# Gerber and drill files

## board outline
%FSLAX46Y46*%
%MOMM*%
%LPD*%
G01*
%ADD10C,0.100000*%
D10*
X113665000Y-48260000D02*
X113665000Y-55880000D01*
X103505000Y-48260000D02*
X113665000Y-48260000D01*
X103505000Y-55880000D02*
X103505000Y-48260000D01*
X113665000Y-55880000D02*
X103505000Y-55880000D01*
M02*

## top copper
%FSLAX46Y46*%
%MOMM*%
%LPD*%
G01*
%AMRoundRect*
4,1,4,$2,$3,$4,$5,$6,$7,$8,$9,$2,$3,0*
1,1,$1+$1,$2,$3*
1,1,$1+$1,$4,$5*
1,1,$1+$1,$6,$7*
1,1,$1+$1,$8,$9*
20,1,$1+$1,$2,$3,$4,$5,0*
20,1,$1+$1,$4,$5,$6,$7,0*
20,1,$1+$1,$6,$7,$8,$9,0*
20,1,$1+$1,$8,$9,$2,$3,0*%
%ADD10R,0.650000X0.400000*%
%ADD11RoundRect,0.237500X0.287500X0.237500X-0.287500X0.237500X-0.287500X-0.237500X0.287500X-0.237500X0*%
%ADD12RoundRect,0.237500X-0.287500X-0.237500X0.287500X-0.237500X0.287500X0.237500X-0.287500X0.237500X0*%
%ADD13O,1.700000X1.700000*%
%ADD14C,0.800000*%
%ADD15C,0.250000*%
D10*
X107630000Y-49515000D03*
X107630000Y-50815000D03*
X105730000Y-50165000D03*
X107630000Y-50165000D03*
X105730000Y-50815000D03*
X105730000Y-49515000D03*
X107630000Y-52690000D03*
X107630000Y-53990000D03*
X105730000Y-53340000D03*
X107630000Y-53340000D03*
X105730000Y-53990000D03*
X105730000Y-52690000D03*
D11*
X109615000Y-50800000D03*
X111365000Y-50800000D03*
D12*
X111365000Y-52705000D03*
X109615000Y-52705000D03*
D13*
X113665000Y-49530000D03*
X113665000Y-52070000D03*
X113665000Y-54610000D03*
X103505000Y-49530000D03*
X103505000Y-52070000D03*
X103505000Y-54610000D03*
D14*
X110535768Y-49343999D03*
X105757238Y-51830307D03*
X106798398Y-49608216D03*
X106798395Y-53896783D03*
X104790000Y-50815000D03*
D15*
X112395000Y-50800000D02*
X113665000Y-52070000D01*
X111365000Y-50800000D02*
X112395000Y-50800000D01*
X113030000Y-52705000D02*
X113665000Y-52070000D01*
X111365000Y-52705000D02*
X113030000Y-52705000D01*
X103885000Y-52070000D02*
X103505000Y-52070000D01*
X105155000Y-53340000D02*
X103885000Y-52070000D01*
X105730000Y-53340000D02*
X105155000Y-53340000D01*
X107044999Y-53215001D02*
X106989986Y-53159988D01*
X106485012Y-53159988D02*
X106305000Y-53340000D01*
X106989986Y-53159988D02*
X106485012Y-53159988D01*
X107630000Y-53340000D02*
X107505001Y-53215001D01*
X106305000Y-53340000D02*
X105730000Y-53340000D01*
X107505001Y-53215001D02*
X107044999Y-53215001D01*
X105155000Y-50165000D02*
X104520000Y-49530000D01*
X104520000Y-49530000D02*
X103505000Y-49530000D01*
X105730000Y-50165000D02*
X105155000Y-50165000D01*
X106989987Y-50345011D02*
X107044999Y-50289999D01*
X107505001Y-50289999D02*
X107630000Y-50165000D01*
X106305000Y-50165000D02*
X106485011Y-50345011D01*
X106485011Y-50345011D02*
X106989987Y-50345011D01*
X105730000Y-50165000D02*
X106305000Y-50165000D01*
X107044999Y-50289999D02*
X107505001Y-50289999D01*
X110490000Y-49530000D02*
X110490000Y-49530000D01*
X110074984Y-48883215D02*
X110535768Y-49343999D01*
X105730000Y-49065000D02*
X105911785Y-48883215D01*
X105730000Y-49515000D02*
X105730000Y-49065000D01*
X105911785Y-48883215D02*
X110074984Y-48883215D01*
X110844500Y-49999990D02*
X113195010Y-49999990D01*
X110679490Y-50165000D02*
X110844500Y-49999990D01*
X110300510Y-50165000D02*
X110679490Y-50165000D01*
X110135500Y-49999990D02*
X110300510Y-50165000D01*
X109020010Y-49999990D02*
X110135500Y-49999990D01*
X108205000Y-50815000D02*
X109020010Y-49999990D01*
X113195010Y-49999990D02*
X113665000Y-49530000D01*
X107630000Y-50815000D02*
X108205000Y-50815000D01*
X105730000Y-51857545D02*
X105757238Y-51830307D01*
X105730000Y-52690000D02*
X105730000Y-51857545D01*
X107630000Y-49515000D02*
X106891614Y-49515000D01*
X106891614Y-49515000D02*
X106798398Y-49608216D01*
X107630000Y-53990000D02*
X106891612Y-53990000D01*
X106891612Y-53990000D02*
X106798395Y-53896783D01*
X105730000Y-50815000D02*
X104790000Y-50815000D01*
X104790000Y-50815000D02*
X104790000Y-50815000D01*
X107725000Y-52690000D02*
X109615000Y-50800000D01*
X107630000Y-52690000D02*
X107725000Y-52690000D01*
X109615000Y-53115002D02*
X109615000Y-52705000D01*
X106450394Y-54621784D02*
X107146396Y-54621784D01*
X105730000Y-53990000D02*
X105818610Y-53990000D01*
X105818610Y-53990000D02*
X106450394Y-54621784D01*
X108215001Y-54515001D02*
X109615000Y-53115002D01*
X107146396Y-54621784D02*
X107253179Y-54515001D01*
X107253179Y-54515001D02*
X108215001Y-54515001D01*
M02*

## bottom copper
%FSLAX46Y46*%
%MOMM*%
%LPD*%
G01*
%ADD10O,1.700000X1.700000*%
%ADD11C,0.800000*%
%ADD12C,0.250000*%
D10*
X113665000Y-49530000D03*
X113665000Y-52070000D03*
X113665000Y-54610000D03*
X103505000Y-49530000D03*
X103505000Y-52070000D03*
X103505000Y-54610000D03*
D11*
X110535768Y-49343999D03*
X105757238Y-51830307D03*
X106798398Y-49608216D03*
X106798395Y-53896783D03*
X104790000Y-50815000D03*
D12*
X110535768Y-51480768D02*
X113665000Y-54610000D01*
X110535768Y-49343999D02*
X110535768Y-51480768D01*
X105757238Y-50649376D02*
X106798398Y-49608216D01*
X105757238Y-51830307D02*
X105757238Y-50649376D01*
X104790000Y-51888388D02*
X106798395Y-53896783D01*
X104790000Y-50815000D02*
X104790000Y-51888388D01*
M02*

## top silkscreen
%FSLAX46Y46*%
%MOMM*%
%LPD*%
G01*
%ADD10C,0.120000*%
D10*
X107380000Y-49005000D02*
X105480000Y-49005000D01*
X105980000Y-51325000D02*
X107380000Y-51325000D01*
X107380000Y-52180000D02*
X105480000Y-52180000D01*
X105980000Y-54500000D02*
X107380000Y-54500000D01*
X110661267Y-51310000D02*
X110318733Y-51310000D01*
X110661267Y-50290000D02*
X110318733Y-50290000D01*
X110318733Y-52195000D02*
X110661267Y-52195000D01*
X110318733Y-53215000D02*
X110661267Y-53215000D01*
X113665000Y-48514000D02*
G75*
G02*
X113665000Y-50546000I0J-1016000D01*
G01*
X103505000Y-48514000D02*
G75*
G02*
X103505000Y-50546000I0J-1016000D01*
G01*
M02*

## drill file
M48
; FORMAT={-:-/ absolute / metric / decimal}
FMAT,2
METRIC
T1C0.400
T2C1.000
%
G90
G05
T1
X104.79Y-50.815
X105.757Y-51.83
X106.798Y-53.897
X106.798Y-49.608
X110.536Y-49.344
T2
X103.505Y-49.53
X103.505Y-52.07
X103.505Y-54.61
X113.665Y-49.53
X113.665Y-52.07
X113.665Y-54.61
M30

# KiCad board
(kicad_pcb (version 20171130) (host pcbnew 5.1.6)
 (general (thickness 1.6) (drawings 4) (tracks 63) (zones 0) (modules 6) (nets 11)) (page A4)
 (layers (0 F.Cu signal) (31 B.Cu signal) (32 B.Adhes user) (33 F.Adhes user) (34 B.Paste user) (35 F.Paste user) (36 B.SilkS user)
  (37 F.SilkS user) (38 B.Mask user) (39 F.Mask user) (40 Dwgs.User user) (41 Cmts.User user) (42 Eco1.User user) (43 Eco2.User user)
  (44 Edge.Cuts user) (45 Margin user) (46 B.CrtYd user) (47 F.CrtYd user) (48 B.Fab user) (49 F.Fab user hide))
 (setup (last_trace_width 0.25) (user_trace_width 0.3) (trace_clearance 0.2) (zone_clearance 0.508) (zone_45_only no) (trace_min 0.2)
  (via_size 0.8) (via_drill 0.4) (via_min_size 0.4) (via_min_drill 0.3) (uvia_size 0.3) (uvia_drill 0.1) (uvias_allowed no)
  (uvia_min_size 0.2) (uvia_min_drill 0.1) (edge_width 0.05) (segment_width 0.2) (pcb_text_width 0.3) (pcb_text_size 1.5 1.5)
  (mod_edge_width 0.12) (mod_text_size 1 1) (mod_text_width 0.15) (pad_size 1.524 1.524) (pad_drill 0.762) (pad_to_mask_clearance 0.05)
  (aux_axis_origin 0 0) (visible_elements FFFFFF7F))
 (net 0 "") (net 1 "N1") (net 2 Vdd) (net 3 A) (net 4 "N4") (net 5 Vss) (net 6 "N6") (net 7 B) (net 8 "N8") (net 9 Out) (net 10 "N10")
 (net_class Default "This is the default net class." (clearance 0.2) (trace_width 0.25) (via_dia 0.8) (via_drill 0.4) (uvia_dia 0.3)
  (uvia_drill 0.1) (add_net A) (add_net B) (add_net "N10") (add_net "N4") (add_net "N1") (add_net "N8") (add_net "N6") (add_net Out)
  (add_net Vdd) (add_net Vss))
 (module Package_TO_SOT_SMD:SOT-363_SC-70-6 (layer F.Cu) (at 106.68 50.165)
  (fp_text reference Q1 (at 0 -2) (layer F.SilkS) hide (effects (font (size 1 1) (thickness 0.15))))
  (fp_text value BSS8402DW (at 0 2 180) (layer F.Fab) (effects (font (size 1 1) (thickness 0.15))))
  (fp_line (start 0.7 -1.16) (end -1.2 -1.16) (layer F.SilkS) (width 0.12))
  (fp_line (start -0.7 1.16) (end 0.7 1.16) (layer F.SilkS) (width 0.12))
  (pad 6 smd rect (at 0.95 -0.65) (size 0.65 0.4) (layers F.Cu F.Paste F.Mask) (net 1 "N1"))
  (pad 4 smd rect (at 0.95 0.65) (size 0.65 0.4) (layers F.Cu F.Paste F.Mask) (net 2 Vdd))
  (pad 2 smd rect (at -0.95 0) (size 0.65 0.4) (layers F.Cu F.Paste F.Mask) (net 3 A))
  (pad 5 smd rect (at 0.95 0) (size 0.65 0.4) (layers F.Cu F.Paste F.Mask) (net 3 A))
  (pad 3 smd rect (at -0.95 0.65) (size 0.65 0.4) (layers F.Cu F.Paste F.Mask) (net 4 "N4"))
  (pad 1 smd rect (at -0.95 -0.65) (size 0.65 0.4) (layers F.Cu F.Paste F.Mask) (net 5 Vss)))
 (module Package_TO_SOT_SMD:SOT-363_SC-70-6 (layer F.Cu) (at 106.68 53.34)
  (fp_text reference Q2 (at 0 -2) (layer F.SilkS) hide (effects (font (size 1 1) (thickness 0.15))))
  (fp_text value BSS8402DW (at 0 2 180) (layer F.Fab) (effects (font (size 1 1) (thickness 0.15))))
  (fp_line (start 0.7 -1.16) (end -1.2 -1.16) (layer F.SilkS) (width 0.12))
  (fp_line (start -0.7 1.16) (end 0.7 1.16) (layer F.SilkS) (width 0.12))
  (pad 6 smd rect (at 0.95 -0.65) (size 0.65 0.4) (layers F.Cu F.Paste F.Mask) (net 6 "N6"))
  (pad 4 smd rect (at 0.95 0.65) (size 0.65 0.4) (layers F.Cu F.Paste F.Mask) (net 4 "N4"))
  (pad 2 smd rect (at -0.95 0) (size 0.65 0.4) (layers F.Cu F.Paste F.Mask) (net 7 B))
  (pad 5 smd rect (at 0.95 0) (size 0.65 0.4) (layers F.Cu F.Paste F.Mask) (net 7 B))
  (pad 3 smd rect (at -0.95 0.65) (size 0.65 0.4) (layers F.Cu F.Paste F.Mask) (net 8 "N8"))
  (pad 1 smd rect (at -0.95 -0.65) (size 0.65 0.4) (layers F.Cu F.Paste F.Mask) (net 1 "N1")))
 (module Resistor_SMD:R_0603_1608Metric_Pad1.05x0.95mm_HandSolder (layer F.Cu) (at 110.49 50.8 180)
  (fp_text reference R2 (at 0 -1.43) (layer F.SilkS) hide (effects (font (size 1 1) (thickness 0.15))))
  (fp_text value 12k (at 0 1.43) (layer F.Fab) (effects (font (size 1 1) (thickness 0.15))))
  (fp_line (start -0.171267 -0.51) (end 0.171267 -0.51) (layer F.SilkS) (width 0.12))
  (fp_line (start -0.171267 0.51) (end 0.171267 0.51) (layer F.SilkS) (width 0.12))
  (pad 2 smd roundrect (at 0.875 0 180) (size 1.05 0.95) (layers F.Cu F.Paste F.Mask) (roundrect_rratio 0.25) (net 6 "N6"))
  (pad 1 smd roundrect (at -0.875 0 180) (size 1.05 0.95) (layers F.Cu F.Paste F.Mask) (roundrect_rratio 0.25) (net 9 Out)))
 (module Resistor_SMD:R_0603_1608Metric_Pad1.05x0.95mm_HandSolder (layer F.Cu) (at 110.49 52.705)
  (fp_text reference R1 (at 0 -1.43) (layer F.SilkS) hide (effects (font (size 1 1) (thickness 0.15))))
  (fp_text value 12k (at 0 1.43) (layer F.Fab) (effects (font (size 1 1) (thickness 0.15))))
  (fp_line (start -0.171267 -0.51) (end 0.171267 -0.51) (layer F.SilkS) (width 0.12))
  (fp_line (start -0.171267 0.51) (end 0.171267 0.51) (layer F.SilkS) (width 0.12))
  (pad 2 smd roundrect (at 0.875 0) (size 1.05 0.95) (layers F.Cu F.Paste F.Mask) (roundrect_rratio 0.25) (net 9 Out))
  (pad 1 smd roundrect (at -0.875 0) (size 1.05 0.95) (layers F.Cu F.Paste F.Mask) (roundrect_rratio 0.25) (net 8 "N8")))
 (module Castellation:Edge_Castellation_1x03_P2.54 (layer F.Cu) (at 113.665 49.53)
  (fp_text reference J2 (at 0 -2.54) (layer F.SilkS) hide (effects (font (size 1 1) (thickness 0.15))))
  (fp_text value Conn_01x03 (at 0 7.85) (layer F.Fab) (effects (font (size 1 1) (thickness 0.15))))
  (fp_arc (start 0 0) (end 0 1.016) (angle -180) (layer F.SilkS) (width 0.12))
  (pad 1 thru_hole oval (at 0 0) (size 1.7 1.7) (drill 1) (layers *.Cu *.Mask) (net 2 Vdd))
  (pad 2 thru_hole oval (at 0 2.54) (size 1.7 1.7) (drill 1) (layers *.Cu *.Mask) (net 9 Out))
  (pad 3 thru_hole oval (at 0 5.08) (size 1.7 1.7) (drill 1) (layers *.Cu *.Mask) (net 5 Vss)))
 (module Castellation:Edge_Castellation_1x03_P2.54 (layer F.Cu) (at 103.505 49.53)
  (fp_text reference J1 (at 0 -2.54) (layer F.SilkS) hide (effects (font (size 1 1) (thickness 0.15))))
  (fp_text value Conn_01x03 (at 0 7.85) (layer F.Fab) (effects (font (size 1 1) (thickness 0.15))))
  (fp_arc (start 0 0) (end 0 1.016) (angle -180) (layer F.SilkS) (width 0.12))
  (pad 1 thru_hole oval (at 0 0) (size 1.7 1.7) (drill 1) (layers *.Cu *.Mask) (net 3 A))
  (pad 2 thru_hole oval (at 0 2.54) (size 1.7 1.7) (drill 1) (layers *.Cu *.Mask) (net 7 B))
  (pad 3 thru_hole oval (at 0 5.08) (size 1.7 1.7) (drill 1) (layers *.Cu *.Mask) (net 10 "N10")))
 (gr_line (start 113.665 48.26) (end 113.665 55.88) (layer Edge.Cuts) (width 0.1))
 (gr_line (start 103.505 48.26) (end 113.665 48.26) (layer Edge.Cuts) (width 0.1))
 (gr_line (start 103.505 55.88) (end 103.505 48.26) (layer Edge.Cuts) (width 0.1))
 (gr_line (start 113.665 55.88) (end 103.505 55.88) (layer Edge.Cuts) (width 0.1))
 (segment (start 112.395 50.8) (end 113.665 52.07) (width 0.25) (layer F.Cu) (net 9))
 (segment (start 111.365 50.8) (end 112.395 50.8) (width 0.25) (layer F.Cu) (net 9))
 (segment (start 113.03 52.705) (end 113.665 52.07) (width 0.25) (layer F.Cu) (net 9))
 (segment (start 111.365 52.705) (end 113.03 52.705) (width 0.25) (layer F.Cu) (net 9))
 (segment (start 103.885 52.07) (end 103.505 52.07) (width 0.25) (layer F.Cu) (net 7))
 (segment (start 105.155 53.34) (end 103.885 52.07) (width 0.25) (layer F.Cu) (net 7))
 (segment (start 105.73 53.34) (end 105.155 53.34) (width 0.25) (layer F.Cu) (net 7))
 (segment (start 107.044999 53.215001) (end 106.989986 53.159988) (width 0.25) (layer F.Cu) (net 7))
 (segment (start 106.485012 53.159988) (end 106.305 53.34) (width 0.25) (layer F.Cu) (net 7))
 (segment (start 106.989986 53.159988) (end 106.485012 53.159988) (width 0.25) (layer F.Cu) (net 7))
 (segment (start 107.63 53.34) (end 107.505001 53.215001) (width 0.25) (layer F.Cu) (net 7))
 (segment (start 106.305 53.34) (end 105.73 53.34) (width 0.25) (layer F.Cu) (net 7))
 (segment (start 107.505001 53.215001) (end 107.044999 53.215001) (width 0.25) (layer F.Cu) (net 7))
 (segment (start 105.155 50.165) (end 104.52 49.53) (width 0.25) (layer F.Cu) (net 3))
 (segment (start 104.52 49.53) (end 103.505 49.53) (width 0.25) (layer F.Cu) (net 3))
 (segment (start 105.73 50.165) (end 105.155 50.165) (width 0.25) (layer F.Cu) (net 3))
 (segment (start 106.989987 50.345011) (end 107.044999 50.289999) (width 0.25) (layer F.Cu) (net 3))
 (segment (start 107.505001 50.289999) (end 107.63 50.165) (width 0.25) (layer F.Cu) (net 3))
 (segment (start 106.305 50.165) (end 106.485011 50.345011) (width 0.25) (layer F.Cu) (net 3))
 (segment (start 106.485011 50.345011) (end 106.989987 50.345011) (width 0.25) (layer F.Cu) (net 3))
 (segment (start 105.73 50.165) (end 106.305 50.165) (width 0.25) (layer F.Cu) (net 3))
 (segment (start 107.044999 50.289999) (end 107.505001 50.289999) (width 0.25) (layer F.Cu) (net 3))
 (segment (start 110.49 49.53) (end 110.49 49.53) (width 0.25) (layer F.Cu) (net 5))
 (via (at 110.535768 49.343999) (size 0.8) (drill 0.4) (layers F.Cu B.Cu) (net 5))
 (segment (start 110.074984 48.883215) (end 110.535768 49.343999) (width 0.25) (layer F.Cu) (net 5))
 (segment (start 105.73 49.065) (end 105.911785 48.883215) (width 0.25) (layer F.Cu) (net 5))
 (segment (start 105.73 49.515) (end 105.73 49.065) (width 0.25) (layer F.Cu) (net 5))
 (segment (start 105.911785 48.883215) (end 110.074984 48.883215) (width 0.25) (layer F.Cu) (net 5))
 (segment (start 110.535768 51.480768) (end 113.665 54.61) (width 0.25) (layer B.Cu) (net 5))
 (segment (start 110.535768 49.343999) (end 110.535768 51.480768) (width 0.25) (layer B.Cu) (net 5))
 (segment (start 110.8445 49.99999) (end 113.19501 49.99999) (width 0.25) (layer F.Cu) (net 2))
 (segment (start 110.67949 50.165) (end 110.8445 49.99999) (width 0.25) (layer F.Cu) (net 2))
 (segment (start 110.30051 50.165) (end 110.67949 50.165) (width 0.25) (layer F.Cu) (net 2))
 (segment (start 110.1355 49.99999) (end 110.30051 50.165) (width 0.25) (layer F.Cu) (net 2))
 (segment (start 109.02001 49.99999) (end 110.1355 49.99999) (width 0.25) (layer F.Cu) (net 2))
 (segment (start 108.205 50.815) (end 109.02001 49.99999) (width 0.25) (layer F.Cu) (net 2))
 (segment (start 113.19501 49.99999) (end 113.665 49.53) (width 0.25) (layer F.Cu) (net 2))
 (segment (start 107.63 50.815) (end 108.205 50.815) (width 0.25) (layer F.Cu) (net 2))
 (via (at 105.757238 51.830307) (size 0.8) (drill 0.4) (layers F.Cu B.Cu) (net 1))
 (segment (start 105.73 51.857545) (end 105.757238 51.830307) (width 0.25) (layer F.Cu) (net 1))
 (segment (start 105.73 52.69) (end 105.73 51.857545) (width 0.25) (layer F.Cu) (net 1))
 (segment (start 107.63 49.515) (end 106.891614 49.515) (width 0.25) (layer F.Cu) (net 1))
 (segment (start 105.757238 50.649376) (end 106.798398 49.608216) (width 0.25) (layer B.Cu) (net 1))
 (segment (start 105.757238 51.830307) (end 105.757238 50.649376) (width 0.25) (layer B.Cu) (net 1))
 (via (at 106.798398 49.608216) (size 0.8) (drill 0.4) (layers F.Cu B.Cu) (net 1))
 (segment (start 106.891614 49.515) (end 106.798398 49.608216) (width 0.25) (layer F.Cu) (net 1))
 (segment (start 107.63 53.99) (end 106.891612 53.99) (width 0.25) (layer F.Cu) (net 4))
 (via (at 106.798395 53.896783) (size 0.8) (drill 0.4) (layers F.Cu B.Cu) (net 4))
 (segment (start 106.891612 53.99) (end 106.798395 53.896783) (width 0.25) (layer F.Cu) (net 4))
 (segment (start 105.73 50.815) (end 104.79 50.815) (width 0.25) (layer F.Cu) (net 4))
 (segment (start 104.79 50.815) (end 104.79 50.815) (width 0.25) (layer F.Cu) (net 4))
 (via (at 104.79 50.815) (size 0.8) (drill 0.4) (layers F.Cu B.Cu) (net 4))
 (segment (start 104.79 51.888388) (end 106.798395 53.896783) (width 0.25) (layer B.Cu) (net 4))
 (segment (start 104.79 50.815) (end 104.79 51.888388) (width 0.25) (layer B.Cu) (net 4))
 (segment (start 107.725 52.69) (end 109.615 50.8) (width 0.25) (layer F.Cu) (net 6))
 (segment (start 107.63 52.69) (end 107.725 52.69) (width 0.25) (layer F.Cu) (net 6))
 (segment (start 109.615 53.115002) (end 109.615 52.705) (width 0.25) (layer F.Cu) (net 8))
 (segment (start 106.450394 54.621784) (end 107.146396 54.621784) (width 0.25) (layer F.Cu) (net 8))
 (segment (start 105.73 53.99) (end 105.81861 53.99) (width 0.25) (layer F.Cu) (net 8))
 (segment (start 105.81861 53.99) (end 106.450394 54.621784) (width 0.25) (layer F.Cu) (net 8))
 (segment (start 108.215001 54.515001) (end 109.615 53.115002) (width 0.25) (layer F.Cu) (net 8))
 (segment (start 107.146396 54.621784) (end 107.253179 54.515001) (width 0.25) (layer F.Cu) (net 8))
 (segment (start 107.253179 54.515001) (end 108.215001 54.515001) (width 0.25) (layer F.Cu) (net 8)))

